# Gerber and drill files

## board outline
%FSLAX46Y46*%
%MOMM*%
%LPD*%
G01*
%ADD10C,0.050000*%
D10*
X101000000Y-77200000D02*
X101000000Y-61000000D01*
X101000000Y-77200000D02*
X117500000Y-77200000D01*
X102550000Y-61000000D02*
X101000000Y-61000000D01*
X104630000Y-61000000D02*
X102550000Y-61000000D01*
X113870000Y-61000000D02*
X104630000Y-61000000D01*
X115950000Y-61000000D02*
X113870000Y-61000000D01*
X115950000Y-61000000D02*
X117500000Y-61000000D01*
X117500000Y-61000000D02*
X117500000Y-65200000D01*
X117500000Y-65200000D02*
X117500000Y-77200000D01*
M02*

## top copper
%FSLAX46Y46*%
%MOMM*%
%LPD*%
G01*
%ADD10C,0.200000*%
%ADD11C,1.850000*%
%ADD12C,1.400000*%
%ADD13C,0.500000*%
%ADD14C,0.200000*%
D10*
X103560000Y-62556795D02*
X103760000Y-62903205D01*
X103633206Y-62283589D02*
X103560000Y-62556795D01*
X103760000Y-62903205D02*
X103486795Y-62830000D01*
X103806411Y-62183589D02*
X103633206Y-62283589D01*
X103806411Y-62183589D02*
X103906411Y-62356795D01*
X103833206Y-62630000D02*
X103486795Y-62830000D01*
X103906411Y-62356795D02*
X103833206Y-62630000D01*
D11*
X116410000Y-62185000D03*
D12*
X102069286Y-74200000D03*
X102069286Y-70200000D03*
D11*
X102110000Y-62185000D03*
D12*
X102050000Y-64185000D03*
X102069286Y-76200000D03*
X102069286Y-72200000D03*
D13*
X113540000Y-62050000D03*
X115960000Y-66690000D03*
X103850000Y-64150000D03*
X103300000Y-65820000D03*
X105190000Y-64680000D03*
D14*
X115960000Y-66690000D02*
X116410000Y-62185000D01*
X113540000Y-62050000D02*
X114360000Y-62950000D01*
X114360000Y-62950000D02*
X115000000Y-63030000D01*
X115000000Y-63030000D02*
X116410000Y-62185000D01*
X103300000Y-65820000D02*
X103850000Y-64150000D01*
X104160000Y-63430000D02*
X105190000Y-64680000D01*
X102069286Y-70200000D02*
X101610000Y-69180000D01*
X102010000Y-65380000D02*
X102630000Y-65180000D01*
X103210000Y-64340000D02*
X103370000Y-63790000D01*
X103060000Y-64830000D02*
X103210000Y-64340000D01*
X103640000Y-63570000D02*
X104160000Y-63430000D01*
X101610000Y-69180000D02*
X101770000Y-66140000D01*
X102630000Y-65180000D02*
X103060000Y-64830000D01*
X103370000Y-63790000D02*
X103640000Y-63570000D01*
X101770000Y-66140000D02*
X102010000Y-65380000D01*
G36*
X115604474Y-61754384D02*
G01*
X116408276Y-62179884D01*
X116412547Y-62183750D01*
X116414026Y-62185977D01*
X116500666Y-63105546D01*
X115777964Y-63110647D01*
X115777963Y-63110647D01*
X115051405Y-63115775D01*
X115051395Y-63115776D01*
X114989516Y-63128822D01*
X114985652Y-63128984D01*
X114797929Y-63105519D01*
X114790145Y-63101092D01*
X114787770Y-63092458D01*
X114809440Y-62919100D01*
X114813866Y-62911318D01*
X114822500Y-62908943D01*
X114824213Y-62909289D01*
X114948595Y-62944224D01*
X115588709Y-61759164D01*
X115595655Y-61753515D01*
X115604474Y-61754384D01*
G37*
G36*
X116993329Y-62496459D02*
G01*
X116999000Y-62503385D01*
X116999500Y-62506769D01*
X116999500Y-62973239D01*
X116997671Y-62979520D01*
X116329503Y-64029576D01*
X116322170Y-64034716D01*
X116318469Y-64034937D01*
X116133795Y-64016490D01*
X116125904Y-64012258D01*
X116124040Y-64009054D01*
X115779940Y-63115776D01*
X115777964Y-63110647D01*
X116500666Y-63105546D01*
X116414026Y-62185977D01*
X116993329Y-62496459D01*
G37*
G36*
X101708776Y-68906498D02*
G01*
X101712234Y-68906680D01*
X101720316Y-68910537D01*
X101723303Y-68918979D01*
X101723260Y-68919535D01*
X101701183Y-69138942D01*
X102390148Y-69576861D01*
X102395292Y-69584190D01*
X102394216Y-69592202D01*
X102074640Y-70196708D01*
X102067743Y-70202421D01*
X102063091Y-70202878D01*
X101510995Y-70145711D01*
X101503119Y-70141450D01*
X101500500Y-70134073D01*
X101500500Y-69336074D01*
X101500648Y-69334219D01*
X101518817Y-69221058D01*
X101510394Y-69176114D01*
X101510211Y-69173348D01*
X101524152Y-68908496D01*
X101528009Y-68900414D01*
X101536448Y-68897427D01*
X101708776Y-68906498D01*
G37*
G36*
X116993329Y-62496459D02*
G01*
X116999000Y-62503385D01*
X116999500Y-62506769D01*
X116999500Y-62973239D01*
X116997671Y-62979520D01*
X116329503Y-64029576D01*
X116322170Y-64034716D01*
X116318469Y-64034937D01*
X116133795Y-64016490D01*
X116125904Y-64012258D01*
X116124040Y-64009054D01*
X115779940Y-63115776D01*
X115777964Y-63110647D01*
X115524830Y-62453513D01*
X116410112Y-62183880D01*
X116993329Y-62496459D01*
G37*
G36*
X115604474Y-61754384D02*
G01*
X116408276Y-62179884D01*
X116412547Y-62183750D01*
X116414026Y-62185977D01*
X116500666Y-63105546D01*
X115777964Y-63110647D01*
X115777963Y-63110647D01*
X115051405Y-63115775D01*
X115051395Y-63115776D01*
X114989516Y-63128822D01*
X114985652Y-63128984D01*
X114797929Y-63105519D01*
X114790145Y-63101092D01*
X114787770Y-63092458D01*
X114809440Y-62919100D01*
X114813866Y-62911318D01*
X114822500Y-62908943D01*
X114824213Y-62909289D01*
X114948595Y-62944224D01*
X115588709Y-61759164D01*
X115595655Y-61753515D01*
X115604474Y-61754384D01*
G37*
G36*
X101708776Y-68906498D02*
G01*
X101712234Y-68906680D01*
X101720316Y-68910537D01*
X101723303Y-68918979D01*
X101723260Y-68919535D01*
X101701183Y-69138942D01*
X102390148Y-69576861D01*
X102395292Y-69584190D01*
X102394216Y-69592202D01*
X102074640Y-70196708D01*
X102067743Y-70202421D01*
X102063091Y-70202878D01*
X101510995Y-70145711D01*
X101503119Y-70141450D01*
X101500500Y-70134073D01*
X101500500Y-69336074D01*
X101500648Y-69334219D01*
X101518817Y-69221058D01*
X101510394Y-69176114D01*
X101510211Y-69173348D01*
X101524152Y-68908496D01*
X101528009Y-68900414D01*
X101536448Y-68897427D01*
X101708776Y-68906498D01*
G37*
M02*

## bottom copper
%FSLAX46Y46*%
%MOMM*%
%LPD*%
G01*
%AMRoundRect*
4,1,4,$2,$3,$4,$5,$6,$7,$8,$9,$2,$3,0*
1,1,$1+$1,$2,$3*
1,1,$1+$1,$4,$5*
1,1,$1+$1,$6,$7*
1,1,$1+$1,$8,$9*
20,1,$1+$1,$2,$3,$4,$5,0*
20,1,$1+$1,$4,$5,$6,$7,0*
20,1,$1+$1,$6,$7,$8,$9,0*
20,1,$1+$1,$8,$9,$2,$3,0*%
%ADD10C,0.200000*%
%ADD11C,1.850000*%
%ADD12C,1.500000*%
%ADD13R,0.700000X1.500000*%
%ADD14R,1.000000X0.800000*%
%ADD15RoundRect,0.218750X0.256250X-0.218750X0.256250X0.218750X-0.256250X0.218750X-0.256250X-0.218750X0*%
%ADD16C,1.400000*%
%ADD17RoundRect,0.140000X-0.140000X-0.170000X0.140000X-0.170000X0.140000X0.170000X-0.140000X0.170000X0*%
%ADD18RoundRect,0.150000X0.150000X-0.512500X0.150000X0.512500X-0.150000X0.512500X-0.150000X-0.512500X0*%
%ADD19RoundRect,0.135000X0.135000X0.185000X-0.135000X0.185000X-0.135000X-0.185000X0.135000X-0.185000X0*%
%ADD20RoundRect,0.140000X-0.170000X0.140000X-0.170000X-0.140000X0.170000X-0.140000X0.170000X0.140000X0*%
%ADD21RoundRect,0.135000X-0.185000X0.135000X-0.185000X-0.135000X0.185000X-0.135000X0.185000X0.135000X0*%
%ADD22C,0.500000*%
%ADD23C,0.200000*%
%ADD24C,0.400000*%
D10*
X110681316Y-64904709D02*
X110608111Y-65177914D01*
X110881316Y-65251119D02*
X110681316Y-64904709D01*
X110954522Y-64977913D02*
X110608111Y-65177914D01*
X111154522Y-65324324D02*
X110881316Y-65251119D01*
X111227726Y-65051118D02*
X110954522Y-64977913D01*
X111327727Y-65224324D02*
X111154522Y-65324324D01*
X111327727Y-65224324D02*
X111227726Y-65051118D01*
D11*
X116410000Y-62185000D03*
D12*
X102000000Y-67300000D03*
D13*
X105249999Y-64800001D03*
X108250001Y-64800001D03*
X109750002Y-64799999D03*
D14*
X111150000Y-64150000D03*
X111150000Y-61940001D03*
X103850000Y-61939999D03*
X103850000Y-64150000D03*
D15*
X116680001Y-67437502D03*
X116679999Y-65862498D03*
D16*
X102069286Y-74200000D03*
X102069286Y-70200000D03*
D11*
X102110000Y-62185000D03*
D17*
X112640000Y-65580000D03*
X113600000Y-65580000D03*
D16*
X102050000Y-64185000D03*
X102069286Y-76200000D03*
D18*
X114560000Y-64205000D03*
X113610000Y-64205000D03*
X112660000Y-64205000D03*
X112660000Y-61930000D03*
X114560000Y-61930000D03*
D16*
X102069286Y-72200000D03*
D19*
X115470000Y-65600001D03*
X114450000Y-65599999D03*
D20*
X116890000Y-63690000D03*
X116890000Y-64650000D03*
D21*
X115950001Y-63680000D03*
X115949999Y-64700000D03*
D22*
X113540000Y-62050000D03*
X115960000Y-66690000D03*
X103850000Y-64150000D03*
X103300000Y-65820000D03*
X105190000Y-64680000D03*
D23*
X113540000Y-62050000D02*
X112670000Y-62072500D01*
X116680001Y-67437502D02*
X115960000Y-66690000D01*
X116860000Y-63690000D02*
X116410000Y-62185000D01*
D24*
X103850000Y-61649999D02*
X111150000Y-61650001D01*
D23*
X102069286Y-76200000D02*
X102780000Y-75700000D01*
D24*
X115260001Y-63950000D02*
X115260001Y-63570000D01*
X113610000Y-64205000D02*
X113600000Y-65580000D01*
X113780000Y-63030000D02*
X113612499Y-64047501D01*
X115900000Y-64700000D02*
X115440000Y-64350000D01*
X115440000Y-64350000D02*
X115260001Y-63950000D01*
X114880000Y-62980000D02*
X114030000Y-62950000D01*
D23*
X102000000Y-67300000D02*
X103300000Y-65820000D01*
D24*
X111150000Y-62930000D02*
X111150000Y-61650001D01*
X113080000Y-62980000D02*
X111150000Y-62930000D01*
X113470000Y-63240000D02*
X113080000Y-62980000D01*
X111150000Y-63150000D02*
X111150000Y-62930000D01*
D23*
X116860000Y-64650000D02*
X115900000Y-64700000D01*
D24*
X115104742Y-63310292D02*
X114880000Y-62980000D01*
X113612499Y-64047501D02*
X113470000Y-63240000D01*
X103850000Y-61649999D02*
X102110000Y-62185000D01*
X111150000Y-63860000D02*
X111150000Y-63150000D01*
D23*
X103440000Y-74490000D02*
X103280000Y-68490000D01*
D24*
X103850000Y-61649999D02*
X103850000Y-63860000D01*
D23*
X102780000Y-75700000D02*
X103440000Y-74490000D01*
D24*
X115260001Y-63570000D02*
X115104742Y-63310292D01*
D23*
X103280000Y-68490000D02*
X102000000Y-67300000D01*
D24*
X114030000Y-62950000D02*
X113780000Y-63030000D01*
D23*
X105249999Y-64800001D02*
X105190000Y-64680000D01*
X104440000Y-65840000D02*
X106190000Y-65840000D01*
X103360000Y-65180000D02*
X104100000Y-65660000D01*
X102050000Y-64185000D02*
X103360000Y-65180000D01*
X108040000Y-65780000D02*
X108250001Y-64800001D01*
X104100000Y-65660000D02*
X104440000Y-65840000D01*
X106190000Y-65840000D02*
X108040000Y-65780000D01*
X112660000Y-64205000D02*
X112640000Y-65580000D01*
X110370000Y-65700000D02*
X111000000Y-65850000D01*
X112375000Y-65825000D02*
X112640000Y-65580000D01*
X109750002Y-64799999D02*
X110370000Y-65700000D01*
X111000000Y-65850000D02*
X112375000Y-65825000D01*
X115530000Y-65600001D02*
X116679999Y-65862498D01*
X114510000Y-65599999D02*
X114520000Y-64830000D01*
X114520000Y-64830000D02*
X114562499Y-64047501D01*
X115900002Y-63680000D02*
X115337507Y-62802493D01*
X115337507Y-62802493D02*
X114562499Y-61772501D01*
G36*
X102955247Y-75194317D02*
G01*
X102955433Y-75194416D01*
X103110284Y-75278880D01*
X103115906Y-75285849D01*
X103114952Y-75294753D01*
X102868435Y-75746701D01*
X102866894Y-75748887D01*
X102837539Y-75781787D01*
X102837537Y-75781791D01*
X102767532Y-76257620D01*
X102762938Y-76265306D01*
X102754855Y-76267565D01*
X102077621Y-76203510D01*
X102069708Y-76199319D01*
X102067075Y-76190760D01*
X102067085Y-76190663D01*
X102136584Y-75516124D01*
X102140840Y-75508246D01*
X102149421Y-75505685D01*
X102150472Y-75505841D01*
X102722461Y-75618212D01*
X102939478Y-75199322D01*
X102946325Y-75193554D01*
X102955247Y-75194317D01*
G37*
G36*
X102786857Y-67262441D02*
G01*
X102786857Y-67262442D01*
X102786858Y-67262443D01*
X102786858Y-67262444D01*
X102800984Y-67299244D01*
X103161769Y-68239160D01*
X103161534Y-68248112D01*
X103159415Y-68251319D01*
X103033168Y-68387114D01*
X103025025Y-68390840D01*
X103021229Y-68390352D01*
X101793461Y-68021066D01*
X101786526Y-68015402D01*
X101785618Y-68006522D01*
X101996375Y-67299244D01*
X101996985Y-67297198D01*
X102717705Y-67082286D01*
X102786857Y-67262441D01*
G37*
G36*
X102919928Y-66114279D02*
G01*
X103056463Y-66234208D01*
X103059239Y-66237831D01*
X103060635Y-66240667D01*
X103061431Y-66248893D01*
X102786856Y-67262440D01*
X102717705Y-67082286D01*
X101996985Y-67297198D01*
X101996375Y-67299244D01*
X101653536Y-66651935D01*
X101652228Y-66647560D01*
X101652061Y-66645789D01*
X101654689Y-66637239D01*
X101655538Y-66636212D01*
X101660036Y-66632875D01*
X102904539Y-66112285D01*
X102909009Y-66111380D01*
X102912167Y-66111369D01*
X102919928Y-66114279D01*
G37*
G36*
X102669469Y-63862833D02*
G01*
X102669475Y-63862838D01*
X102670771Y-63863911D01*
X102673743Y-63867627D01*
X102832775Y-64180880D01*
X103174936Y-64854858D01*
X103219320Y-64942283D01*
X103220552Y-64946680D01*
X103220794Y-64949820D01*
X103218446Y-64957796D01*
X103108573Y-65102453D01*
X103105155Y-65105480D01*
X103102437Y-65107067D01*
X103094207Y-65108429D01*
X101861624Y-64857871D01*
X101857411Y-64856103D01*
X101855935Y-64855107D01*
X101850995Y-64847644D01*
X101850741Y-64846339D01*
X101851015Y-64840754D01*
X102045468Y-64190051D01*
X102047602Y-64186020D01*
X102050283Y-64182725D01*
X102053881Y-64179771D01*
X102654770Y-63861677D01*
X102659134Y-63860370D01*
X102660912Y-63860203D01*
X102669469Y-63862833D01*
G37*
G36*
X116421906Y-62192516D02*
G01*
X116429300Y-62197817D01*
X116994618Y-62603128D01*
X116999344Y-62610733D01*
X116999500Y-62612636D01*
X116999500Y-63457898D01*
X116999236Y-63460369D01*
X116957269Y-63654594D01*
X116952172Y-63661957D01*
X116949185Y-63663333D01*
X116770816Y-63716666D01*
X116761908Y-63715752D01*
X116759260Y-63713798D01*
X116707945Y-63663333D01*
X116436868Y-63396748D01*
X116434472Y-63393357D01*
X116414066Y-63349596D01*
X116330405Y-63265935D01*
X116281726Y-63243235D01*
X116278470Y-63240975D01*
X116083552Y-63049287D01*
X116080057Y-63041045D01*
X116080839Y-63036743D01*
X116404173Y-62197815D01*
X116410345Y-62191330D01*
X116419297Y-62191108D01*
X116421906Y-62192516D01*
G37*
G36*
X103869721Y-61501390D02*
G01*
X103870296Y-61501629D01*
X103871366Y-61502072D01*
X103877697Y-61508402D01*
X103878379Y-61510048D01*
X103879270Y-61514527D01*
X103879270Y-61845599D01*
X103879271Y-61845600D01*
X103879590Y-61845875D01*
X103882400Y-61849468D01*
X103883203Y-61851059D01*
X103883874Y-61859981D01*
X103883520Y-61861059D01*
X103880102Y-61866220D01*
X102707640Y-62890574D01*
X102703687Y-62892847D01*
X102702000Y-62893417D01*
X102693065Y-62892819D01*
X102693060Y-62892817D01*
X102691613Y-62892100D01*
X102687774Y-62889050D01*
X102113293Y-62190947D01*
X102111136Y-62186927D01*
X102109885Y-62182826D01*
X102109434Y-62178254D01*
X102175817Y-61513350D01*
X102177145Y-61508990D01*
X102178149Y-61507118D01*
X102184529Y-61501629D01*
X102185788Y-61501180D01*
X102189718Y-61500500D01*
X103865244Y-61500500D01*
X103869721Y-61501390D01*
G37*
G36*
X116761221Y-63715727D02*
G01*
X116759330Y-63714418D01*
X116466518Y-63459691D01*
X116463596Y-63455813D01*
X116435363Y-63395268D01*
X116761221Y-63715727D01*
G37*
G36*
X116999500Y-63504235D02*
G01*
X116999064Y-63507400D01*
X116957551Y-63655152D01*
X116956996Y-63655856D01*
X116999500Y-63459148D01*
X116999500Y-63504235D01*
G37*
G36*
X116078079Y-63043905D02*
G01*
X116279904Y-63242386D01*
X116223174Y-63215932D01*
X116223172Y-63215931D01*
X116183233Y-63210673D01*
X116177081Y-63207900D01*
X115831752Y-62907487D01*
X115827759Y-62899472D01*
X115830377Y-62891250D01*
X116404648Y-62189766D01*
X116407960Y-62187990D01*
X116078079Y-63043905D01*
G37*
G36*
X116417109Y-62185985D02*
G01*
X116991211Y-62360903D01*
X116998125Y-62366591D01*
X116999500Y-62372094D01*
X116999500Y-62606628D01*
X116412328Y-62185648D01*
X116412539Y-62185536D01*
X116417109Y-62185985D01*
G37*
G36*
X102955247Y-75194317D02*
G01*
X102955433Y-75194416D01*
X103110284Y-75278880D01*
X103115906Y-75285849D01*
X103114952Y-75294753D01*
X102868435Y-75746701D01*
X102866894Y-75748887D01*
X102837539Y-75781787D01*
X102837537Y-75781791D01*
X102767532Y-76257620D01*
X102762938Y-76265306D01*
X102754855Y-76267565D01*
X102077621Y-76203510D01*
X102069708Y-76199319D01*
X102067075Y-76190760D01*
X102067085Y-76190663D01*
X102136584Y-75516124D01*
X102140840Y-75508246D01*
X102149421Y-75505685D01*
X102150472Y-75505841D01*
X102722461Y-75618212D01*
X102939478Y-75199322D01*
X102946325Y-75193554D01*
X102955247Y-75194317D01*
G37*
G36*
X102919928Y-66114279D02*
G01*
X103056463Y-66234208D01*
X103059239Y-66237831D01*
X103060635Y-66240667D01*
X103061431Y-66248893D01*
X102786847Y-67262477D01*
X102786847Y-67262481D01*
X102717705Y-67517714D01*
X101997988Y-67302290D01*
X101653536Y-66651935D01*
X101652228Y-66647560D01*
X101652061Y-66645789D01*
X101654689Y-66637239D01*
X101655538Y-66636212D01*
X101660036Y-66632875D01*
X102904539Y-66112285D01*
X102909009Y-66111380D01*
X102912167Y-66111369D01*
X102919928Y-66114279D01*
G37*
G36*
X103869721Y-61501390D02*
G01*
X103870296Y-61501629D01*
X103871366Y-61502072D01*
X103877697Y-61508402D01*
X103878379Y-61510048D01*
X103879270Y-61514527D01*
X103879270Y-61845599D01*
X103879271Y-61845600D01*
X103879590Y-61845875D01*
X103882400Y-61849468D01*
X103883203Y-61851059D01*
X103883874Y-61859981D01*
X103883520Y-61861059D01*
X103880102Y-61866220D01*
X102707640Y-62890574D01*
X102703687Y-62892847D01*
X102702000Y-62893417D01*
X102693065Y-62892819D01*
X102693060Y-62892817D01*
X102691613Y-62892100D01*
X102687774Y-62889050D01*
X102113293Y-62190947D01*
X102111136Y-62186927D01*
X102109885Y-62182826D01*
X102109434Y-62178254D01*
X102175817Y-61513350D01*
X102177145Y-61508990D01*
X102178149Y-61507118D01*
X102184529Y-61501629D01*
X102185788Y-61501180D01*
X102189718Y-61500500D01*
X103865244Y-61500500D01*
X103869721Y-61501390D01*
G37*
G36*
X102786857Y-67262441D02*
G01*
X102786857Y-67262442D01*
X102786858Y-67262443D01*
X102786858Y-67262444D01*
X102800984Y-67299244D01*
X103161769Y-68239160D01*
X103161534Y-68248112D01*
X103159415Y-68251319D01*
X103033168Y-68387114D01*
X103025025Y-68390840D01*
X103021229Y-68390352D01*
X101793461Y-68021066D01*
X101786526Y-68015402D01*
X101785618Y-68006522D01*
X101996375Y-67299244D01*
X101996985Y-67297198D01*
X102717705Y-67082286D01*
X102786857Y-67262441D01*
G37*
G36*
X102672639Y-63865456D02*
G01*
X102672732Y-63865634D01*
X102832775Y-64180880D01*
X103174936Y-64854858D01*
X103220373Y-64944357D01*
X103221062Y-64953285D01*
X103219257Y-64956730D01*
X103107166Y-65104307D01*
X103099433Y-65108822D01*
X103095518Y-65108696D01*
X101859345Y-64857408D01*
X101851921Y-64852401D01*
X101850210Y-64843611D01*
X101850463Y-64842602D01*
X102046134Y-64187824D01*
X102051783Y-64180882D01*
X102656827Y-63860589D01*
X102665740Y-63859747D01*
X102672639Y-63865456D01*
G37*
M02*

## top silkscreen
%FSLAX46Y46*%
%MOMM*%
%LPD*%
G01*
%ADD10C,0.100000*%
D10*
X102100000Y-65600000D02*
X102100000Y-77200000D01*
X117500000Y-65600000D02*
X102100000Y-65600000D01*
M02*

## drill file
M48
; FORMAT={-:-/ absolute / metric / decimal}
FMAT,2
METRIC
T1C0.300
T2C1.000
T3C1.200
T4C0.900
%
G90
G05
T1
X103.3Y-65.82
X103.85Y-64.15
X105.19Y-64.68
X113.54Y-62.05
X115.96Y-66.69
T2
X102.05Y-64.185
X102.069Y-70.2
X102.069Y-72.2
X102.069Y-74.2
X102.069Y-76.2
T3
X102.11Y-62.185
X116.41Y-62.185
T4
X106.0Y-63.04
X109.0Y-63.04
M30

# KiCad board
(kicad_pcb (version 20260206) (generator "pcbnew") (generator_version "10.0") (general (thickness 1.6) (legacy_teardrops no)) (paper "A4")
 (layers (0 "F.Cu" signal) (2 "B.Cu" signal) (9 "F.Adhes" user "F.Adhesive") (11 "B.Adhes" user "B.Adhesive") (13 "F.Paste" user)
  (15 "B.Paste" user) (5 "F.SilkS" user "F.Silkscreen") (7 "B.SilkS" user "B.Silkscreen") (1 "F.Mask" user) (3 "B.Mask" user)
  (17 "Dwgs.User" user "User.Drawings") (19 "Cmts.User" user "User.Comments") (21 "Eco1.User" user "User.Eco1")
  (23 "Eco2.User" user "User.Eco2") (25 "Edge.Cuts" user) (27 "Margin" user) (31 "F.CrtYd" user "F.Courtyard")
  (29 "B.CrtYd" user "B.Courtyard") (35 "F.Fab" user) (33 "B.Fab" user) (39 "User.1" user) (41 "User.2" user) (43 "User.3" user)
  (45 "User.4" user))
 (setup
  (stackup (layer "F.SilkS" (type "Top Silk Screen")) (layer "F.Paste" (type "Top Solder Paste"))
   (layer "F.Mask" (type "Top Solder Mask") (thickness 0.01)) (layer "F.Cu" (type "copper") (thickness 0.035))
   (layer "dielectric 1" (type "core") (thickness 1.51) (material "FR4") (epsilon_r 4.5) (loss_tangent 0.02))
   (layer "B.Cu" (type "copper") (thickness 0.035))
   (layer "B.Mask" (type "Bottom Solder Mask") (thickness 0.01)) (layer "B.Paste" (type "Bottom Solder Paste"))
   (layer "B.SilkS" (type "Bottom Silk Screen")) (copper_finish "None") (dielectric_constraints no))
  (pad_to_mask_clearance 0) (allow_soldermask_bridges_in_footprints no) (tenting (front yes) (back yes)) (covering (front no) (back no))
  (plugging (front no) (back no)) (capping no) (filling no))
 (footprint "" (layer "F.Cu") (at 116.41 62.185)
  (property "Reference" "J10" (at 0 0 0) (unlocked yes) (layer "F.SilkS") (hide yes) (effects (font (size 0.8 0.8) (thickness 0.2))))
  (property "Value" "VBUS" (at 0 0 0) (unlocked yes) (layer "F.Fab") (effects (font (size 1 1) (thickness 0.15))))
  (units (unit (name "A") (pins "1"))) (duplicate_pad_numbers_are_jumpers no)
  (pad "1" thru_hole circle (at 0 0 180) (size 1.85 1.85) (drill 1.2) (layers "*.Cu" "*.Mask") (remove_unused_layers no) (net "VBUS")
   (teardrops (best_length_ratio 0.5) (max_length 1) (best_width_ratio 1) (max_width 2) (curved_edges no) (filter_ratio 0.9) (enabled yes)
    (allow_two_segments yes) (prefer_zone_connections yes))))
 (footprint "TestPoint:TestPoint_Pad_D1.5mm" (layer "B.Cu") (at 102 67.3 180)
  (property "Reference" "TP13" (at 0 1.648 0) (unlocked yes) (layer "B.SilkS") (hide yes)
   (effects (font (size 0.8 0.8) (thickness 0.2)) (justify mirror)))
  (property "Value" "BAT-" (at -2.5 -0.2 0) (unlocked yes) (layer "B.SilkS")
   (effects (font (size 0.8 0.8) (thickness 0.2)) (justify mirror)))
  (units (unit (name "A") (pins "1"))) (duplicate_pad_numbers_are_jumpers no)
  (pad "1" smd circle (at 0 0 180) (size 1.5 1.5) (layers "B.Cu" "B.Mask") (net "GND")
   (teardrops (best_length_ratio 0.5) (max_length 1) (best_width_ratio 1) (max_width 2) (curved_edges no) (filter_ratio 0.9) (enabled yes)
    (allow_two_segments yes) (prefer_zone_connections yes))))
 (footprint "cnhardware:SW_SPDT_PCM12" (layer "B.Cu") (at 107.5 63.37)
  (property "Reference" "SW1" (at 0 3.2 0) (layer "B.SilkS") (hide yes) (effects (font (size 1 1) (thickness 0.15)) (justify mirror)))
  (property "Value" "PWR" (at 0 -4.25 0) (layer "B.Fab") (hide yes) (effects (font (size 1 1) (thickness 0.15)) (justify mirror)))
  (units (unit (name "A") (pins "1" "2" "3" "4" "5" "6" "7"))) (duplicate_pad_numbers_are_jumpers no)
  (pad "" np_thru_hole circle (at -1.5 -0.33) (size 0.9 0.9) (drill 0.9) (layers "*.Cu" "*.Mask"))
  (pad "" np_thru_hole circle (at 1.5 -0.33) (size 0.9 0.9) (drill 0.9) (layers "*.Cu" "*.Mask"))
  (pad "1" smd rect (at -2.250001 1.430001) (size 0.7 1.5) (layers "B.Cu" "B.Mask" "B.Paste") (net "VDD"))
  (pad "2" smd rect (at 0.750001 1.430001) (size 0.7 1.5) (layers "B.Cu" "B.Mask" "B.Paste") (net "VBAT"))
  (pad "3" smd rect (at 2.250002 1.429999) (size 0.7 1.5) (layers "B.Cu" "B.Mask" "B.Paste") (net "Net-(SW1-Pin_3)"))
  (pad "4" smd rect (at 3.65 0.78) (size 1 0.8) (layers "B.Cu" "B.Mask" "B.Paste") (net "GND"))
  (pad "5" smd rect (at 3.65 -1.429999) (size 1 0.8) (layers "B.Cu" "B.Mask" "B.Paste") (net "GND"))
  (pad "6" smd rect (at -3.65 -1.430001) (size 1 0.8) (layers "B.Cu" "B.Mask" "B.Paste") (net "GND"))
  (pad "7" smd rect (at -3.65 0.78) (size 1 0.8) (layers "B.Cu" "B.Mask" "B.Paste") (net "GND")))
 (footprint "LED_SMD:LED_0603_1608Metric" (layer "B.Cu") (at 116.68 66.65 90)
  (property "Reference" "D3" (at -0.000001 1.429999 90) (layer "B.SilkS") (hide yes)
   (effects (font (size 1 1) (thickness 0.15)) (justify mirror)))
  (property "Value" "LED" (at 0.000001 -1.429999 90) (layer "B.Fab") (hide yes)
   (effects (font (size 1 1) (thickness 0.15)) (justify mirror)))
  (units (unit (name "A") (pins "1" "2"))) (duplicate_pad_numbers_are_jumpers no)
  (pad "1" smd roundrect (at -0.787502 0.000001 90) (size 0.875 0.95) (layers "B.Cu" "B.Mask" "B.Paste") (roundrect_rratio 0.25)
   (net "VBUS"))
  (pad "2" smd roundrect (at 0.787502 -0.000001 90) (size 0.875 0.95) (layers "B.Cu" "B.Mask" "B.Paste") (roundrect_rratio 0.25)
   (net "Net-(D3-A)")))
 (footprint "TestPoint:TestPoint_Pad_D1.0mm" (layer "B.Cu") (at 102.069286 74.2 180)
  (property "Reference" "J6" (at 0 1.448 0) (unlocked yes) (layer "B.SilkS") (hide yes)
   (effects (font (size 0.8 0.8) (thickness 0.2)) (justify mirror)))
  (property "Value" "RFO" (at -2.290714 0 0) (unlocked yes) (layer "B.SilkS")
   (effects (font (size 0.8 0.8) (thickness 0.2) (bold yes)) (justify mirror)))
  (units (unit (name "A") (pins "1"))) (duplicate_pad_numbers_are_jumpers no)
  (pad "1" thru_hole circle (at 0 0 180) (size 1.4 1.4) (drill 1) (layers "*.Cu" "*.Mask") (remove_unused_layers no)
   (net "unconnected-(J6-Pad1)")
   (teardrops (best_length_ratio 0.5) (max_length 1) (best_width_ratio 1) (max_width 2) (curved_edges no) (filter_ratio 0.9) (enabled yes)
    (allow_two_segments yes) (prefer_zone_connections yes))))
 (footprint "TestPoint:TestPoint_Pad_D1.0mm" (layer "B.Cu") (at 102.069286 70.2 180)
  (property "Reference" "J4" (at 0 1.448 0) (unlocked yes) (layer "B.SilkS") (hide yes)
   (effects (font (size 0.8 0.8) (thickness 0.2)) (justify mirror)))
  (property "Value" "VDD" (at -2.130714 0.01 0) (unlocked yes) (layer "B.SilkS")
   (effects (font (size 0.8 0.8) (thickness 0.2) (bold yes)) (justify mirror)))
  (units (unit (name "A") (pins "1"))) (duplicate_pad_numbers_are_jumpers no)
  (pad "1" thru_hole circle (at 0 0 180) (size 1.4 1.4) (drill 1) (layers "*.Cu" "*.Mask") (remove_unused_layers no) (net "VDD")
   (teardrops (best_length_ratio 0.5) (max_length 1) (best_width_ratio 1) (max_width 2) (curved_edges no) (filter_ratio 0.9) (enabled yes)
    (allow_two_segments yes) (prefer_zone_connections yes))))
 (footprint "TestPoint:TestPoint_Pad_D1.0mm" (layer "B.Cu") (at 102.11 62.185 180)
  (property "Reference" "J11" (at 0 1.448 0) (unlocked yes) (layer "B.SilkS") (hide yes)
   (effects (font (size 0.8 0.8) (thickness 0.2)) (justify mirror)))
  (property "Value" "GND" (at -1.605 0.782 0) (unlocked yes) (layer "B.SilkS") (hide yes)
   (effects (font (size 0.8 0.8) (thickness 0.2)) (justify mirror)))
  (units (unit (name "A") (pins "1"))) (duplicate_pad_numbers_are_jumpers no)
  (pad "1" thru_hole circle (at 0 0 180) (size 1.85 1.85) (drill 1.2) (layers "*.Cu" "*.Mask") (remove_unused_layers no) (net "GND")
   (teardrops (best_length_ratio 0.5) (max_length 1) (best_width_ratio 1) (max_width 2) (curved_edges no) (filter_ratio 0.9) (enabled yes)
    (allow_two_segments yes) (prefer_zone_connections yes))))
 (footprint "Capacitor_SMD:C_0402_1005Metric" (layer "B.Cu") (at 113.12 65.58)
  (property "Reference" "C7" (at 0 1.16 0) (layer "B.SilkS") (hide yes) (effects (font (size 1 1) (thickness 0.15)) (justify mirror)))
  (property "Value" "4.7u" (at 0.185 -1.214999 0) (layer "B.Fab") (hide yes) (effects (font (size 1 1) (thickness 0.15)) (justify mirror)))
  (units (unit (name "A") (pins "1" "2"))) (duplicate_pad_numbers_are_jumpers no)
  (pad "1" smd roundrect (at -0.48 0) (size 0.56 0.62) (layers "B.Cu" "B.Mask" "B.Paste") (roundrect_rratio 0.25) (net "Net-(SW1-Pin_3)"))
  (pad "2" smd roundrect (at 0.48 0) (size 0.56 0.62) (layers "B.Cu" "B.Mask" "B.Paste") (roundrect_rratio 0.25) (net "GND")))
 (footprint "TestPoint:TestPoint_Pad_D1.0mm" (layer "B.Cu") (at 102.05 64.185 180)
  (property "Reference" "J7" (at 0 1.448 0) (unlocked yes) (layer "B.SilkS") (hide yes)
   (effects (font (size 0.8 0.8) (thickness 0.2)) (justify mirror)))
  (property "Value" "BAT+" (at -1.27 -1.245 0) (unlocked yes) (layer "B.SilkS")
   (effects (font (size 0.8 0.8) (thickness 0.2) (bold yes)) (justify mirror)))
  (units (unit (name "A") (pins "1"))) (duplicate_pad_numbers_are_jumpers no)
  (pad "1" thru_hole circle (at 0 0 180) (size 1.4 1.4) (drill 1) (layers "*.Cu" "*.Mask") (remove_unused_layers no) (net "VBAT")
   (teardrops (best_length_ratio 0.5) (max_length 1) (best_width_ratio 1) (max_width 2) (curved_edges no) (filter_ratio 0.9) (enabled yes)
    (allow_two_segments yes) (prefer_zone_connections yes))))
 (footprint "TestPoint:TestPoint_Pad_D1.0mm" (layer "B.Cu") (at 102.069286 76.2 180)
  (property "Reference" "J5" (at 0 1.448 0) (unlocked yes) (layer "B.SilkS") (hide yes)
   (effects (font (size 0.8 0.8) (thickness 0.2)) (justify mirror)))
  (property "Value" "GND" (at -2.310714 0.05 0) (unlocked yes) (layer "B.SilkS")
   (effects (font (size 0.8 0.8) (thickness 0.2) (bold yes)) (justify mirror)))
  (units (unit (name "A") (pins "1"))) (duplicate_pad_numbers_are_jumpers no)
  (pad "1" thru_hole circle (at 0 0 180) (size 1.4 1.4) (drill 1) (layers "*.Cu" "*.Mask") (remove_unused_layers no) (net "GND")
   (teardrops (best_length_ratio 0.5) (max_length 1) (best_width_ratio 1) (max_width 2) (curved_edges no) (filter_ratio 0.9) (enabled yes)
    (allow_two_segments yes) (prefer_zone_connections yes))))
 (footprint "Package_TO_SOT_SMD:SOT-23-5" (layer "B.Cu") (at 113.61 63.0675 90)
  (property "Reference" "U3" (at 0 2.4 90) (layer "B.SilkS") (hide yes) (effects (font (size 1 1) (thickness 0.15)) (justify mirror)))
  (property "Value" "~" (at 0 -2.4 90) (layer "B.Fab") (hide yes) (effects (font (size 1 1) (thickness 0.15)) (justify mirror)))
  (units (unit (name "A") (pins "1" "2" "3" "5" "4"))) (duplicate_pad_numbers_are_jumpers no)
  (pad "1" smd roundrect (at -1.1375 0.95 90) (size 1.325 0.6) (layers "B.Cu" "B.Mask" "B.Paste") (roundrect_rratio 0.25)
   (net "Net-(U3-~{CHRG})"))
  (pad "2" smd roundrect (at -1.1375 0 90) (size 1.325 0.6) (layers "B.Cu" "B.Mask" "B.Paste") (roundrect_rratio 0.25) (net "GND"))
  (pad "3" smd roundrect (at -1.1375 -0.95 90) (size 1.325 0.6) (layers "B.Cu" "B.Mask" "B.Paste") (roundrect_rratio 0.25)
   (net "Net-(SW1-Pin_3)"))
  (pad "4" smd roundrect (at 1.1375 -0.95 90) (size 1.325 0.6) (layers "B.Cu" "B.Mask" "B.Paste") (roundrect_rratio 0.25) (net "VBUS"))
  (pad "5" smd roundrect (at 1.1375 0.95 90) (size 1.325 0.6) (layers "B.Cu" "B.Mask" "B.Paste") (roundrect_rratio 0.25)
   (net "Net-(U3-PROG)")))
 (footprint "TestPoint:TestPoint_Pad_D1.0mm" (layer "B.Cu") (at 102.069286 72.2 180)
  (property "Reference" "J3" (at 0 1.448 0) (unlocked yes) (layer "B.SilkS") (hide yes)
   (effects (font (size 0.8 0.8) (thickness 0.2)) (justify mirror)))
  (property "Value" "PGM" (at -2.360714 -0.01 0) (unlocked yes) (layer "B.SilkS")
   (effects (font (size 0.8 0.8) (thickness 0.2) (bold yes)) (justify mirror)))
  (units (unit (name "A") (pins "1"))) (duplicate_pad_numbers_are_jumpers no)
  (pad "1" thru_hole circle (at 0 0 180) (size 1.4 1.4) (drill 1) (layers "*.Cu" "*.Mask") (remove_unused_layers no)
   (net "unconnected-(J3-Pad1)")
   (teardrops (best_length_ratio 0.5) (max_length 1) (best_width_ratio 1) (max_width 2) (curved_edges no) (filter_ratio 0.9) (enabled yes)
    (allow_two_segments yes) (prefer_zone_connections yes))))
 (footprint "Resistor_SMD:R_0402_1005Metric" (layer "B.Cu") (at 114.96 65.6 180)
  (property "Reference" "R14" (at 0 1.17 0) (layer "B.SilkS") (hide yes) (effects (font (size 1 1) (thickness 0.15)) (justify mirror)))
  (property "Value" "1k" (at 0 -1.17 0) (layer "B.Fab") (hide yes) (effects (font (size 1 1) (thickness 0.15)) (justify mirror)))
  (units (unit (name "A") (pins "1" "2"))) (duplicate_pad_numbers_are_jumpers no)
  (pad "1" smd roundrect (at -0.51 -0.000001 180) (size 0.54 0.64) (layers "B.Cu" "B.Mask" "B.Paste") (roundrect_rratio 0.25)
   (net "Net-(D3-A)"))
  (pad "2" smd roundrect (at 0.51 0.000001 180) (size 0.54 0.64) (layers "B.Cu" "B.Mask" "B.Paste") (roundrect_rratio 0.25)
   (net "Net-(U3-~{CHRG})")))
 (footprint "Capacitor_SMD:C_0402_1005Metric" (layer "B.Cu") (at 116.89 64.17 -90)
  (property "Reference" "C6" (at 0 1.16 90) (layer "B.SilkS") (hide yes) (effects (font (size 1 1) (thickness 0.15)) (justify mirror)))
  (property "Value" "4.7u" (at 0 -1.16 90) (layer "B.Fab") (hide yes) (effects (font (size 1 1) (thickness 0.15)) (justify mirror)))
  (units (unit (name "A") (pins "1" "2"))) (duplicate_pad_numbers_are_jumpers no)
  (pad "1" smd roundrect (at -0.48 0 270) (size 0.56 0.62) (layers "B.Cu" "B.Mask" "B.Paste") (roundrect_rratio 0.25) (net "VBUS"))
  (pad "2" smd roundrect (at 0.48 0 270) (size 0.56 0.62) (layers "B.Cu" "B.Mask" "B.Paste") (roundrect_rratio 0.25) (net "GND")))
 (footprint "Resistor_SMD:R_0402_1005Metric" (layer "B.Cu") (at 115.95 64.19 -90)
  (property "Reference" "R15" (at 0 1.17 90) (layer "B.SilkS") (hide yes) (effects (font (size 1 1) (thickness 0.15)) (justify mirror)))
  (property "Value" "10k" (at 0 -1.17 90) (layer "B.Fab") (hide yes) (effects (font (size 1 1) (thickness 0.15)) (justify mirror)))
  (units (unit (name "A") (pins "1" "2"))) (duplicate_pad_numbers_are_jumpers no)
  (pad "1" smd roundrect (at -0.51 -0.000001 270) (size 0.54 0.64) (layers "B.Cu" "B.Mask" "B.Paste") (roundrect_rratio 0.25)
   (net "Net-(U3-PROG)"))
  (pad "2" smd roundrect (at 0.51 0.000001 270) (size 0.54 0.64) (layers "B.Cu" "B.Mask" "B.Paste") (roundrect_rratio 0.25) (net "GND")))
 (gr_line (start 103.56 62.556795) (end 103.76 62.903205) (stroke (width 0.2) (type default)) (layer "F.Cu"))
 (gr_line (start 103.633206 62.283589) (end 103.56 62.556795) (stroke (width 0.2) (type default)) (layer "F.Cu"))
 (gr_line (start 103.76 62.903205) (end 103.486795 62.83) (stroke (width 0.2) (type default)) (layer "F.Cu"))
 (gr_line (start 103.806411 62.183589) (end 103.633206 62.283589) (stroke (width 0.2) (type default)) (layer "F.Cu"))
 (gr_line (start 103.806411 62.183589) (end 103.906411 62.356795) (stroke (width 0.2) (type default)) (layer "F.Cu"))
 (gr_line (start 103.833206 62.63) (end 103.486795 62.83) (stroke (width 0.2) (type default)) (layer "F.Cu"))
 (gr_line (start 103.906411 62.356795) (end 103.833206 62.63) (stroke (width 0.2) (type default)) (layer "F.Cu"))
 (gr_line (start 110.681316 64.904709) (end 110.608111 65.177914) (stroke (width 0.2) (type default)) (layer "B.Cu"))
 (gr_line (start 110.881316 65.251119) (end 110.681316 64.904709) (stroke (width 0.2) (type default)) (layer "B.Cu"))
 (gr_line (start 110.954522 64.977913) (end 110.608111 65.177914) (stroke (width 0.2) (type default)) (layer "B.Cu"))
 (gr_line (start 111.154522 65.324324) (end 110.881316 65.251119) (stroke (width 0.2) (type default)) (layer "B.Cu"))
 (gr_line (start 111.227726 65.051118) (end 110.954522 64.977913) (stroke (width 0.2) (type default)) (layer "B.Cu"))
 (gr_line (start 111.327727 65.224324) (end 111.154522 65.324324) (stroke (width 0.2) (type default)) (layer "B.Cu"))
 (gr_line (start 111.327727 65.224324) (end 111.227726 65.051118) (stroke (width 0.2) (type default)) (layer "B.Cu"))
 (gr_line (start 102.1 65.6) (end 102.1 77.2) (stroke (width 0.1) (type default)) (layer "F.SilkS"))
 (gr_line (start 117.5 65.6) (end 102.1 65.6) (stroke (width 0.1) (type default)) (layer "F.SilkS"))
 (gr_line (start 101 77.2) (end 101 61) (stroke (width 0.05) (type default)) (layer "Edge.Cuts"))
 (gr_line (start 101 77.2) (end 117.5 77.2) (stroke (width 0.05) (type default)) (layer "Edge.Cuts"))
 (gr_line (start 102.55 61) (end 101 61) (stroke (width 0.05) (type default)) (layer "Edge.Cuts"))
 (gr_line (start 104.63 61) (end 102.55 61) (stroke (width 0.05) (type solid)) (layer "Edge.Cuts"))
 (gr_line (start 113.87 61) (end 104.63 61) (stroke (width 0.05) (type default)) (layer "Edge.Cuts"))
 (gr_line (start 115.95 61) (end 113.87 61) (stroke (width 0.05) (type solid)) (layer "Edge.Cuts"))
 (gr_line (start 115.95 61) (end 117.5 61) (stroke (width 0.05) (type default)) (layer "Edge.Cuts"))
 (gr_line (start 117.5 61) (end 117.5 65.2) (stroke (width 0.05) (type solid)) (layer "Edge.Cuts"))
 (gr_line (start 117.5 65.2) (end 117.5 77.2) (stroke (width 0.05) (type default)) (layer "Edge.Cuts"))
 (segment (start 115.96 66.69) (end 116.41 62.185) (width 0.2) (layer "F.Cu") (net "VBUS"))
 (segment (start 113.54 62.05) (end 114.36 62.95) (width 0.2) (layer "F.Cu") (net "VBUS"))
 (segment (start 114.36 62.95) (end 115 63.03) (width 0.2) (layer "F.Cu") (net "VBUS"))
 (segment (start 115 63.03) (end 116.41 62.185) (width 0.2) (layer "F.Cu") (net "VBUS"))
 (via (at 113.54 62.05) (size 0.5) (drill 0.3) (layers "F.Cu" "B.Cu") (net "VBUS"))
 (via (at 115.96 66.69) (size 0.5) (drill 0.3) (layers "F.Cu" "B.Cu") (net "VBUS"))
 (segment (start 113.54 62.05) (end 112.67 62.0725) (width 0.2) (layer "B.Cu") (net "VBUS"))
 (segment (start 116.680001 67.437502) (end 115.96 66.69) (width 0.2) (layer "B.Cu") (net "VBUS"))
 (segment (start 116.86 63.69) (end 116.41 62.185) (width 0.2) (layer "B.Cu") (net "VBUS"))
 (segment (start 103.3 65.82) (end 103.85 64.15) (width 0.2) (layer "F.Cu") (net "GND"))
 (via (at 103.85 64.15) (size 0.5) (drill 0.3) (layers "F.Cu" "B.Cu") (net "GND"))
 (via (at 103.3 65.82) (size 0.5) (drill 0.3) (layers "F.Cu" "B.Cu") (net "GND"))
 (segment (start 103.85 61.649999) (end 111.15 61.650001) (width 0.4) (layer "B.Cu") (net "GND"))
 (segment (start 102.069286 76.2) (end 102.78 75.7) (width 0.2) (layer "B.Cu") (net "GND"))
 (segment (start 115.260001 63.95) (end 115.260001 63.57) (width 0.4) (layer "B.Cu") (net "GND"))
 (segment (start 113.61 64.205) (end 113.6 65.58) (width 0.4) (layer "B.Cu") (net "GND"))
 (segment (start 113.78 63.03) (end 113.612499 64.047501) (width 0.4) (layer "B.Cu") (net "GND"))
 (segment (start 115.9 64.7) (end 115.44 64.35) (width 0.4) (layer "B.Cu") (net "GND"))
 (segment (start 115.44 64.35) (end 115.260001 63.95) (width 0.4) (layer "B.Cu") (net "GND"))
 (segment (start 114.88 62.98) (end 114.03 62.95) (width 0.4) (layer "B.Cu") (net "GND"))
 (segment (start 102 67.3) (end 103.3 65.82) (width 0.2) (layer "B.Cu") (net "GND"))
 (segment (start 111.15 62.93) (end 111.15 61.650001) (width 0.4) (layer "B.Cu") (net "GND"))
 (segment (start 113.08 62.98) (end 111.15 62.93) (width 0.4) (layer "B.Cu") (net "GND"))
 (segment (start 113.47 63.24) (end 113.08 62.98) (width 0.4) (layer "B.Cu") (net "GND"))
 (segment (start 111.15 63.15) (end 111.15 62.93) (width 0.4) (layer "B.Cu") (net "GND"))
 (segment (start 116.86 64.65) (end 115.9 64.7) (width 0.2) (layer "B.Cu") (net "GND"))
 (segment (start 115.104742 63.310292) (end 114.88 62.98) (width 0.4) (layer "B.Cu") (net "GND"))
 (segment (start 113.612499 64.047501) (end 113.47 63.24) (width 0.4) (layer "B.Cu") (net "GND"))
 (segment (start 103.85 61.649999) (end 102.11 62.185) (width 0.4) (layer "B.Cu") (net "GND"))
 (segment (start 111.15 63.86) (end 111.15 63.15) (width 0.4) (layer "B.Cu") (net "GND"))
 (segment (start 103.44 74.49) (end 103.28 68.49) (width 0.2) (layer "B.Cu") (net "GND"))
 (segment (start 103.85 61.649999) (end 103.85 63.86) (width 0.4) (layer "B.Cu") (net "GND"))
 (segment (start 102.78 75.7) (end 103.44 74.49) (width 0.2) (layer "B.Cu") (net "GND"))
 (segment (start 115.260001 63.57) (end 115.104742 63.310292) (width 0.4) (layer "B.Cu") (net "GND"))
 (segment (start 103.28 68.49) (end 102 67.3) (width 0.2) (layer "B.Cu") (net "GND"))
 (segment (start 114.03 62.95) (end 113.78 63.03) (width 0.4) (layer "B.Cu") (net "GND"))
 (segment (start 104.16 63.43) (end 105.19 64.68) (width 0.2) (layer "F.Cu") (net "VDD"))
 (segment (start 102.069286 70.2) (end 101.61 69.18) (width 0.2) (layer "F.Cu") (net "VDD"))
 (segment (start 102.01 65.38) (end 102.63 65.18) (width 0.2) (layer "F.Cu") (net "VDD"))
 (segment (start 103.21 64.34) (end 103.37 63.79) (width 0.2) (layer "F.Cu") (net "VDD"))
 (segment (start 103.06 64.83) (end 103.21 64.34) (width 0.2) (layer "F.Cu") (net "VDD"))
 (segment (start 103.64 63.57) (end 104.16 63.43) (width 0.2) (layer "F.Cu") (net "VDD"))
 (segment (start 101.61 69.18) (end 101.77 66.14) (width 0.2) (layer "F.Cu") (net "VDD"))
 (segment (start 102.63 65.18) (end 103.06 64.83) (width 0.2) (layer "F.Cu") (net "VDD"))
 (segment (start 103.37 63.79) (end 103.64 63.57) (width 0.2) (layer "F.Cu") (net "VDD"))
 (segment (start 101.77 66.14) (end 102.01 65.38) (width 0.2) (layer "F.Cu") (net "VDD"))
 (via (at 105.19 64.68) (size 0.5) (drill 0.3) (layers "F.Cu" "B.Cu") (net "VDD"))
 (segment (start 105.249999 64.800001) (end 105.19 64.68) (width 0.2) (layer "B.Cu") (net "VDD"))
 (segment (start 104.44 65.84) (end 106.19 65.84) (width 0.2) (layer "B.Cu") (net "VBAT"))
 (segment (start 103.36 65.18) (end 104.1 65.66) (width 0.2) (layer "B.Cu") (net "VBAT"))
 (segment (start 102.05 64.185) (end 103.36 65.18) (width 0.2) (layer "B.Cu") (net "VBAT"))
 (segment (start 108.04 65.78) (end 108.250001 64.800001) (width 0.2) (layer "B.Cu") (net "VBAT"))
 (segment (start 104.1 65.66) (end 104.44 65.84) (width 0.2) (layer "B.Cu") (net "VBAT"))
 (segment (start 106.19 65.84) (end 108.04 65.78) (width 0.2) (layer "B.Cu") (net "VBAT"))
 (segment (start 112.66 64.205) (end 112.64 65.58) (width 0.2) (layer "B.Cu") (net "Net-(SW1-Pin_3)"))
 (segment (start 110.37 65.7) (end 111 65.85) (width 0.2) (layer "B.Cu") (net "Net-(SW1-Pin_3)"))
 (segment (start 112.375 65.825) (end 112.64 65.58) (width 0.2) (layer "B.Cu") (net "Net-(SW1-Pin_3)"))
 (segment (start 109.750002 64.799999) (end 110.37 65.7) (width 0.2) (layer "B.Cu") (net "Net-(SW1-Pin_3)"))
 (segment (start 111 65.85) (end 112.375 65.825) (width 0.2) (layer "B.Cu") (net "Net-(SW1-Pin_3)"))
 (segment (start 115.53 65.600001) (end 116.679999 65.862498) (width 0.2) (layer "B.Cu") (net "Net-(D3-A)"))
 (segment (start 114.51 65.599999) (end 114.52 64.83) (width 0.2) (layer "B.Cu") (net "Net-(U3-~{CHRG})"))
 (segment (start 114.52 64.83) (end 114.562499 64.047501) (width 0.2) (layer "B.Cu") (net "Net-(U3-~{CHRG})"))
 (segment (start 115.900002 63.68) (end 115.337507 62.802493) (width 0.2) (layer "B.Cu") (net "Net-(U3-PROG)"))
 (segment (start 115.337507 62.802493) (end 114.562499 61.772501) (width 0.2) (layer "B.Cu") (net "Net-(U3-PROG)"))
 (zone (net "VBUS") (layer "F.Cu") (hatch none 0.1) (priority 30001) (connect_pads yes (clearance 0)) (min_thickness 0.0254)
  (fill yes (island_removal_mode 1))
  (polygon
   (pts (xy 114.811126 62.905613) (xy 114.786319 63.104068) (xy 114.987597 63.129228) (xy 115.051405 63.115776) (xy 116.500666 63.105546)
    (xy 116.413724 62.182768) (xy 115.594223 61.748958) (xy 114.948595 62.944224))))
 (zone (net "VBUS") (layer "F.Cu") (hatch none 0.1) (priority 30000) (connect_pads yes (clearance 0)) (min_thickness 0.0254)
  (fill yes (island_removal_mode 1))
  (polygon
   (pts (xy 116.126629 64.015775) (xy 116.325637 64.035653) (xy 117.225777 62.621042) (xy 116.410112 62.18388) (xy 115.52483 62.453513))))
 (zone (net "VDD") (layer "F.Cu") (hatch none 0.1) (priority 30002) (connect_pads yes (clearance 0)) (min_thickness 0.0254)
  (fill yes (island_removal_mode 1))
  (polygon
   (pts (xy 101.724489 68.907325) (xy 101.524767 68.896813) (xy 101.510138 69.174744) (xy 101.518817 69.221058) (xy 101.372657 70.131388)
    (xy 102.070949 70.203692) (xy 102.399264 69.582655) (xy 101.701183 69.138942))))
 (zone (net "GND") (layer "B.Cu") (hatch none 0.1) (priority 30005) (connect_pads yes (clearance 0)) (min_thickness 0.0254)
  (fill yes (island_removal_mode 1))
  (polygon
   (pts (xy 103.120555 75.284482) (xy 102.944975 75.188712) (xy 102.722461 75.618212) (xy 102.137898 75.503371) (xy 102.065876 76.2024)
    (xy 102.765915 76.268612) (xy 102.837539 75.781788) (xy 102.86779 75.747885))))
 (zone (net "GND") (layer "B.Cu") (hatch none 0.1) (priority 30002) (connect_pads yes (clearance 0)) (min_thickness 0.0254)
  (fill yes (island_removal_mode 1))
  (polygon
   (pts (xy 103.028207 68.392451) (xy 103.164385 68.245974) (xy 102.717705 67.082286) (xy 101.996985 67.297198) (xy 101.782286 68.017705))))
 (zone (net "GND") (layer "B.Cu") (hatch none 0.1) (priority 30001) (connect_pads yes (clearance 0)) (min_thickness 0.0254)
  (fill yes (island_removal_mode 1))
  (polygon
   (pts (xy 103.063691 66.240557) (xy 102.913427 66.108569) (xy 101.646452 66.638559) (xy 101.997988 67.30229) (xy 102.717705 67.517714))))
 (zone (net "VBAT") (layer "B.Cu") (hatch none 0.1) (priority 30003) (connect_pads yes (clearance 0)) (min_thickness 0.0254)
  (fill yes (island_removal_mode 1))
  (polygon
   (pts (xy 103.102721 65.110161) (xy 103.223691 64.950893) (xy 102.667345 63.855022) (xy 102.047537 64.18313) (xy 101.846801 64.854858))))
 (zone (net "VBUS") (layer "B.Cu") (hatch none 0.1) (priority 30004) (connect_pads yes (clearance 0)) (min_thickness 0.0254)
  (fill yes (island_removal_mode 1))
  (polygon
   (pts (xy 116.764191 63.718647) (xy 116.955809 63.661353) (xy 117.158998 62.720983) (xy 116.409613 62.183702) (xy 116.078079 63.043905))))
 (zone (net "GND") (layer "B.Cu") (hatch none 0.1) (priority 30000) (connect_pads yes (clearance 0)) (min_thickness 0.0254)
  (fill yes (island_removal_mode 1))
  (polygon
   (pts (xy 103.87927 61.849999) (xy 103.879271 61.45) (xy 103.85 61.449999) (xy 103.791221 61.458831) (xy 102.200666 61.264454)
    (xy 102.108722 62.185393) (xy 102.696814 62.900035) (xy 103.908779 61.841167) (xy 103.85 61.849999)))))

